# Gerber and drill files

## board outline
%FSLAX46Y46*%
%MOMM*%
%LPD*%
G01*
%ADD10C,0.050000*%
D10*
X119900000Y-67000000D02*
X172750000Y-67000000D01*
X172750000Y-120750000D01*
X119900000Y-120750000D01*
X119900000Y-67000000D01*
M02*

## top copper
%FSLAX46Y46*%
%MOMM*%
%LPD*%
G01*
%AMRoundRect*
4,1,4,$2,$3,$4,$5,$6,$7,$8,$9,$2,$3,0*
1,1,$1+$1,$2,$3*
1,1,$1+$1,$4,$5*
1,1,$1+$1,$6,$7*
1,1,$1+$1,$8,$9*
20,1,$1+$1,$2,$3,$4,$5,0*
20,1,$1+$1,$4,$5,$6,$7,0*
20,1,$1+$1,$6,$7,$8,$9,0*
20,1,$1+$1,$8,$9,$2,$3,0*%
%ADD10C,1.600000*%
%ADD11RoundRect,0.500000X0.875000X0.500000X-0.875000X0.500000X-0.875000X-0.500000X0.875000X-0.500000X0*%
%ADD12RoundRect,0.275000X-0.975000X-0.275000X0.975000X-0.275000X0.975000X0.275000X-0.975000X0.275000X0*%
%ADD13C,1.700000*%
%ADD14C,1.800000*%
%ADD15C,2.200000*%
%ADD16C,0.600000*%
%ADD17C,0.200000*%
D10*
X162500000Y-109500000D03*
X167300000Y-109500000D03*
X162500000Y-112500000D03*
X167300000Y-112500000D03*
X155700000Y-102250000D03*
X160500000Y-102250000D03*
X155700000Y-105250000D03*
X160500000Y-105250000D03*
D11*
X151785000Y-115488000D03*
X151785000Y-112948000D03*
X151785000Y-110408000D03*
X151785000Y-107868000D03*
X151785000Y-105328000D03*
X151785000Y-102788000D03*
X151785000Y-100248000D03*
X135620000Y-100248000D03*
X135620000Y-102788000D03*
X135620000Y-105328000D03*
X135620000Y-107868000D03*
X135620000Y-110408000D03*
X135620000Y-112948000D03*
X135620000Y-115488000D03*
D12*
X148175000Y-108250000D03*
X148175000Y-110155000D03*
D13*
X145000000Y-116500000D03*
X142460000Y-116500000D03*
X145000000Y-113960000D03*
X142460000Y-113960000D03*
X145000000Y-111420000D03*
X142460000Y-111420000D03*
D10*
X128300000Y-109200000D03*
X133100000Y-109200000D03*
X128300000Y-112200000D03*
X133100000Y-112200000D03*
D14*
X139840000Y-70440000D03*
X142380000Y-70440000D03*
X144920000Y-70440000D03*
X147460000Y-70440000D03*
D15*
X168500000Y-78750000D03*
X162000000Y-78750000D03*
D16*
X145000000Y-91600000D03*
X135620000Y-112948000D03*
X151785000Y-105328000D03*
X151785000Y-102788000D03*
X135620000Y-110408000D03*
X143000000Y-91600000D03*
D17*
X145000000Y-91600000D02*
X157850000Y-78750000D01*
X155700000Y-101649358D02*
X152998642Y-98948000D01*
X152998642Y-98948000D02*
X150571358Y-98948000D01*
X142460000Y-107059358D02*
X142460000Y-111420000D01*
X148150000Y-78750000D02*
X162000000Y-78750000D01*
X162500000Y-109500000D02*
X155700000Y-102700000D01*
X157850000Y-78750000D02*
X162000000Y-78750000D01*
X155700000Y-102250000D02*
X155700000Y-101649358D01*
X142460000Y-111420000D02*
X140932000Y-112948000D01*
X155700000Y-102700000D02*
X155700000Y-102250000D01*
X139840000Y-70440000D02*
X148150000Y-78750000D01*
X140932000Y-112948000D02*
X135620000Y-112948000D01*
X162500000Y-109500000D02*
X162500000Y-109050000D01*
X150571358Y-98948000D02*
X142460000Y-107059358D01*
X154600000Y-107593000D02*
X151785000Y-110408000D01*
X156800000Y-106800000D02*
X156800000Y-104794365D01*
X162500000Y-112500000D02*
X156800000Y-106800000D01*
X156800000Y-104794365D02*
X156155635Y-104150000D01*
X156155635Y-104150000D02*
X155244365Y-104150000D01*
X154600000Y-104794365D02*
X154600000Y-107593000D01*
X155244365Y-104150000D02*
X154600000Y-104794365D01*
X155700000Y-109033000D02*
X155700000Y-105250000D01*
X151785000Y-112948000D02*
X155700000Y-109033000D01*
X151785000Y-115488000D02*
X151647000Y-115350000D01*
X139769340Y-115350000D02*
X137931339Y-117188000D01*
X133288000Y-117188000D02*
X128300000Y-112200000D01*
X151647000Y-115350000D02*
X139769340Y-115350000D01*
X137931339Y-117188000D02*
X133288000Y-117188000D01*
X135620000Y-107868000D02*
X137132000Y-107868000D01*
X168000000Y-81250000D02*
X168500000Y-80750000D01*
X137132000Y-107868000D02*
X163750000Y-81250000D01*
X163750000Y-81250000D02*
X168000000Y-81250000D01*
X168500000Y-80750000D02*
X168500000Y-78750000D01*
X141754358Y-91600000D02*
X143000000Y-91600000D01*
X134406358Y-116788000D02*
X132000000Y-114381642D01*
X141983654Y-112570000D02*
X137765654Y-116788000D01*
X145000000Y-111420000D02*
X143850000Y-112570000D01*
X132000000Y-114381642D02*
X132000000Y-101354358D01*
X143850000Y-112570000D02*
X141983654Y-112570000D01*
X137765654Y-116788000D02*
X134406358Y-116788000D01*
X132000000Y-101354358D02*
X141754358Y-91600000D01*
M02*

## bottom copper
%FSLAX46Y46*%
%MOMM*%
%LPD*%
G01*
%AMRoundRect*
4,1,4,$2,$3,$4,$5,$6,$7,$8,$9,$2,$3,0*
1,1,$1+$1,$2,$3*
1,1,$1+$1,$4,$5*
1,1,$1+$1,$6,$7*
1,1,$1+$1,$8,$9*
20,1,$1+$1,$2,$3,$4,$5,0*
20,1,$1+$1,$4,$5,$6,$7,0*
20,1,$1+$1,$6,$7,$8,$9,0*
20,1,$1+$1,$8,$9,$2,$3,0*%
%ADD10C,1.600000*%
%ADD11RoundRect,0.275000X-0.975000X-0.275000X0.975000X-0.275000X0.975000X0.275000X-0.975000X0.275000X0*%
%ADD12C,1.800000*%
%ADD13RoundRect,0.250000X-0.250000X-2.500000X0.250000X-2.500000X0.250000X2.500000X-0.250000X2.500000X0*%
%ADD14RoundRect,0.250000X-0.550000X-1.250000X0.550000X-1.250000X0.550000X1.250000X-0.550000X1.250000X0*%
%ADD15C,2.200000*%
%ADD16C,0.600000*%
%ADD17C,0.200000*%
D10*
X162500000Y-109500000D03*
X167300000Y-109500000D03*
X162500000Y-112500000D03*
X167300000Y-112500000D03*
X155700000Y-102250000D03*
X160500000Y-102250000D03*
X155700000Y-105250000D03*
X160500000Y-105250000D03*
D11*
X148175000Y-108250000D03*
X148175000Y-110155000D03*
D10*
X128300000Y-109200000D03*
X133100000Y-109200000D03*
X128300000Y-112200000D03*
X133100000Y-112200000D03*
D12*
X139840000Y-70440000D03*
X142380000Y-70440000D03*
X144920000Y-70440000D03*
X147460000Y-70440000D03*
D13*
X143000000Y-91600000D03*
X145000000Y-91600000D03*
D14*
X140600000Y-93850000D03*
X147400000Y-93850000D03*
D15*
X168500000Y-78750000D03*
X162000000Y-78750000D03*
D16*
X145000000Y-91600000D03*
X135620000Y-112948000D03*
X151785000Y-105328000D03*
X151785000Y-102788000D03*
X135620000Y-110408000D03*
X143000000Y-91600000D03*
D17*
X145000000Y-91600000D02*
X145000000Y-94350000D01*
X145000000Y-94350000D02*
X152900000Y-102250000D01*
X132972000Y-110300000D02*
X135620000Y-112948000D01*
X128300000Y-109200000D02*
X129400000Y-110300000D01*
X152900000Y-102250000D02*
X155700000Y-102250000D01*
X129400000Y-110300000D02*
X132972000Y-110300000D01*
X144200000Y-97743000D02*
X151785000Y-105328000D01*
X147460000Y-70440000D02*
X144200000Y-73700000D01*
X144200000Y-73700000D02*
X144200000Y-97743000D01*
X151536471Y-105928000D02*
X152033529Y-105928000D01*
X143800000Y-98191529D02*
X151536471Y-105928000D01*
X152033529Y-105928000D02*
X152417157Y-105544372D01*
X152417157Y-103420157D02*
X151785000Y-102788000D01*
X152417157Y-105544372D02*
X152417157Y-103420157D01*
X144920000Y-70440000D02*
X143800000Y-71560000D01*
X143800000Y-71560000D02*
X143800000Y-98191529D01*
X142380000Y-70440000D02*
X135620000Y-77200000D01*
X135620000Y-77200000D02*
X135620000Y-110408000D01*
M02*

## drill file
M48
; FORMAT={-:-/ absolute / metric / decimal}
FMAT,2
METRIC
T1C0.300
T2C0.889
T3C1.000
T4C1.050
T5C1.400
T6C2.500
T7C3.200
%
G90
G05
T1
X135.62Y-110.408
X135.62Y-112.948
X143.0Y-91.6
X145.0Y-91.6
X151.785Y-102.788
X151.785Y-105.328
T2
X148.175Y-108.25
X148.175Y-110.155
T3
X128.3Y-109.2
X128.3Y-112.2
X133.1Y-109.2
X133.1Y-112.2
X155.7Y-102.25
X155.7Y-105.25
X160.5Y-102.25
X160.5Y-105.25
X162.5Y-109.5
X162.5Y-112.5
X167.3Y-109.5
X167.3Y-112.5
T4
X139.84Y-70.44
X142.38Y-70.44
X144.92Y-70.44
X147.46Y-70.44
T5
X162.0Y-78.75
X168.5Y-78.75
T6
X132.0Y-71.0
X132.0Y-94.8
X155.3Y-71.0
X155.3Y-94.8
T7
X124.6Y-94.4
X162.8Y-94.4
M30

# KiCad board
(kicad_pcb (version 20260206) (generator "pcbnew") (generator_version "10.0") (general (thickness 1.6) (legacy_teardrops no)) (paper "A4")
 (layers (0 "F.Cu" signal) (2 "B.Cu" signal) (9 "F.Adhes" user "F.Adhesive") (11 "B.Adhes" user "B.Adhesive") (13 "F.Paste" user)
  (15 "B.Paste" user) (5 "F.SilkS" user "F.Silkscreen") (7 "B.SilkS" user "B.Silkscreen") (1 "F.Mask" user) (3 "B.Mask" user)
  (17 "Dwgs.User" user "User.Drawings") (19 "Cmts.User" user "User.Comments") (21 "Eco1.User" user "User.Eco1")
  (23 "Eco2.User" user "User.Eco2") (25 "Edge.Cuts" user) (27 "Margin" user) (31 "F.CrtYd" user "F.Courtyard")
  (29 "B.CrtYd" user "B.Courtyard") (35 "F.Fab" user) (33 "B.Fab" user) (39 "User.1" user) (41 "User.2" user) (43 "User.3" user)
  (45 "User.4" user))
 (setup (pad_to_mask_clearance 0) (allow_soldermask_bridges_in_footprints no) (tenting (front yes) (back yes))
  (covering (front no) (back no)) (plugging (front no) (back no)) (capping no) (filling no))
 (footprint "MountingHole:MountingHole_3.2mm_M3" (layer "F.Cu") (at 162.8 94.4)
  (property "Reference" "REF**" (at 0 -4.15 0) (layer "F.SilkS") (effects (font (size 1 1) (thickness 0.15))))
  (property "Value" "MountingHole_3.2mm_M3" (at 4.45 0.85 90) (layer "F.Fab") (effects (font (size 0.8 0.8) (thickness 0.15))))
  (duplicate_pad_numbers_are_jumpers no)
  (pad "" np_thru_hole circle (at 0 0) (size 3.2 3.2) (drill 3.2) (layers "*.Cu" "*.Mask")))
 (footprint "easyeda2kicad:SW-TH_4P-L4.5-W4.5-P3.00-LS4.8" (layer "F.Cu") (at 164.9 111)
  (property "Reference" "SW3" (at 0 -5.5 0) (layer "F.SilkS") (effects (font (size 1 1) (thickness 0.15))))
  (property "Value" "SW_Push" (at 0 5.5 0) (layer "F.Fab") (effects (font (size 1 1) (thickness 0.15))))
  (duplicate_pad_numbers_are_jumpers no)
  (pad "1" thru_hole circle (at -2.4 -1.5) (size 1.6 1.6) (drill 0.999998) (layers "*.Cu" "*.Mask") (remove_unused_layers no) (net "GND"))
  (pad "1" thru_hole circle (at 2.4 -1.5) (size 1.6 1.6) (drill 0.999998) (layers "*.Cu" "*.Mask") (remove_unused_layers no))
  (pad "2" thru_hole circle (at -2.4 1.5) (size 1.6 1.6) (drill 0.999998) (layers "*.Cu" "*.Mask") (remove_unused_layers no)
   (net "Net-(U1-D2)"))
  (pad "2" thru_hole circle (at 2.4 1.5) (size 1.6 1.6) (drill 0.999998) (layers "*.Cu" "*.Mask") (remove_unused_layers no)))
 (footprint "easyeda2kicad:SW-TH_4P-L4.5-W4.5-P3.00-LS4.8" (layer "F.Cu") (at 158.1 103.75)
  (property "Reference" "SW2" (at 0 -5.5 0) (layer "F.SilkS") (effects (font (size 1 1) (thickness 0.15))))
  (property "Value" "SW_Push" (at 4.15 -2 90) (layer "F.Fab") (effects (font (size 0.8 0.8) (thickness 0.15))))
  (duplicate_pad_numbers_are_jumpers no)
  (pad "1" thru_hole circle (at -2.4 -1.5) (size 1.6 1.6) (drill 0.999998) (layers "*.Cu" "*.Mask") (remove_unused_layers no) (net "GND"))
  (pad "1" thru_hole circle (at 2.4 -1.5) (size 1.6 1.6) (drill 0.999998) (layers "*.Cu" "*.Mask") (remove_unused_layers no))
  (pad "2" thru_hole circle (at -2.4 1.5) (size 1.6 1.6) (drill 0.999998) (layers "*.Cu" "*.Mask") (remove_unused_layers no)
   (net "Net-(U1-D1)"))
  (pad "2" thru_hole circle (at 2.4 1.5) (size 1.6 1.6) (drill 0.999998) (layers "*.Cu" "*.Mask") (remove_unused_layers no)))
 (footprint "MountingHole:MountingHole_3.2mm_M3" (layer "F.Cu") (at 124.6 94.4)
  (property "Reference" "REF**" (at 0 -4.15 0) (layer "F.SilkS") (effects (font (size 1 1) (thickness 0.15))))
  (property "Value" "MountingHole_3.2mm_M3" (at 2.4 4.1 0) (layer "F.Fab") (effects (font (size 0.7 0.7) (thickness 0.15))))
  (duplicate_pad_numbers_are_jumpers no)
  (pad "" np_thru_hole circle (at 0 0) (size 3.2 3.2) (drill 3.2) (layers "*.Cu" "*.Mask")))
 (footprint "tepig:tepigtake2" (layer "F.Cu") (at 124.75 74.25)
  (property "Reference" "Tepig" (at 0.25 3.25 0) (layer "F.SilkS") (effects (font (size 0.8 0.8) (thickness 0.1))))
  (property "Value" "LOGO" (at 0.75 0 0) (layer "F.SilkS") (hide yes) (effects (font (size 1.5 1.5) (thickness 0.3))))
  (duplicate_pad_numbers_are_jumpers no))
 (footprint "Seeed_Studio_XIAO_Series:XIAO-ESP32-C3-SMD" (layer "F.Cu") (at 152.62 97.368 180)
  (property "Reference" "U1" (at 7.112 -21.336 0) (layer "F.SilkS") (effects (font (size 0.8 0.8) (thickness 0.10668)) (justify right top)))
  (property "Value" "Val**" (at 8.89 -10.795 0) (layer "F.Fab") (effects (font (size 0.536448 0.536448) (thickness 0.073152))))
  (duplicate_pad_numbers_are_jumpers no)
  (pad "1" smd roundrect (at 0.835 -18.12 180) (size 2.75 2) (layers "F.Cu" "F.Mask" "F.Paste") (roundrect_rratio 0.25) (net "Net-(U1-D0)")
   (solder_mask_margin 0.0508) (thermal_bridge_angle 45))
  (pad "2" smd roundrect (at 0.835 -15.58 180) (size 2.75 2) (layers "F.Cu" "F.Mask" "F.Paste") (roundrect_rratio 0.25) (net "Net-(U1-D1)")
   (solder_mask_margin 0.0508) (thermal_bridge_angle 45))
  (pad "3" smd roundrect (at 0.835 -13.04 180) (size 2.75 2) (layers "F.Cu" "F.Mask" "F.Paste") (roundrect_rratio 0.25) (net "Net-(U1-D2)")
   (solder_mask_margin 0.0508) (thermal_bridge_angle 45))
  (pad "4" smd roundrect (at 0.835 -10.5 180) (size 2.75 2) (layers "F.Cu" "F.Mask" "F.Paste") (roundrect_rratio 0.25)
   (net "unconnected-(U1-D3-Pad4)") (solder_mask_margin 0.0508) (thermal_bridge_angle 45))
  (pad "5" smd roundrect (at 0.835 -7.96 180) (size 2.75 2) (layers "F.Cu" "F.Mask" "F.Paste") (roundrect_rratio 0.25) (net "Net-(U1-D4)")
   (solder_mask_margin 0.0508) (thermal_bridge_angle 45))
  (pad "6" smd roundrect (at 0.835 -5.42 180) (size 2.75 2) (layers "F.Cu" "F.Mask" "F.Paste") (roundrect_rratio 0.25) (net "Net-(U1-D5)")
   (solder_mask_margin 0.0508) (thermal_bridge_angle 45))
  (pad "7" smd roundrect (at 0.835 -2.88 180) (size 2.75 2) (layers "F.Cu" "F.Mask" "F.Paste") (roundrect_rratio 0.25)
   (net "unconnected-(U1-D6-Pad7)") (solder_mask_margin 0.0508) (thermal_bridge_angle 45))
  (pad "8" smd roundrect (at 17 -2.88 180) (size 2.75 2) (layers "F.Cu" "F.Mask" "F.Paste") (roundrect_rratio 0.25)
   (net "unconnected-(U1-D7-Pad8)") (solder_mask_margin 0.0508) (thermal_bridge_angle 45))
  (pad "9" smd roundrect (at 17 -5.42 180) (size 2.75 2) (layers "F.Cu" "F.Mask" "F.Paste") (roundrect_rratio 0.25)
   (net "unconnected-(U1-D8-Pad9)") (solder_mask_margin 0.0508) (thermal_bridge_angle 45))
  (pad "10" smd roundrect (at 17 -7.96 180) (size 2.75 2) (layers "F.Cu" "F.Mask" "F.Paste") (roundrect_rratio 0.25)
   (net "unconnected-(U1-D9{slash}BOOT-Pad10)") (solder_mask_margin 0.0508) (thermal_bridge_angle 45))
  (pad "11" smd roundrect (at 17 -10.5 180) (size 2.75 2) (layers "F.Cu" "F.Mask" "F.Paste") (roundrect_rratio 0.25) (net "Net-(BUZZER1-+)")
   (solder_mask_margin 0.0508) (thermal_bridge_angle 45))
  (pad "12" smd roundrect (at 17 -13.04 180) (size 2.75 2) (layers "F.Cu" "F.Mask" "F.Paste") (roundrect_rratio 0.25) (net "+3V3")
   (solder_mask_margin 0.0508) (thermal_bridge_angle 45))
  (pad "13" smd roundrect (at 17 -15.58 180) (size 2.75 2) (layers "F.Cu" "F.Mask" "F.Paste") (roundrect_rratio 0.25) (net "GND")
   (solder_mask_margin 0.0508) (thermal_bridge_angle 45))
  (pad "14" smd roundrect (at 17 -18.12 180) (size 2.75 2) (layers "F.Cu" "F.Mask" "F.Paste") (roundrect_rratio 0.25) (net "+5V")
   (solder_mask_margin 0.0508) (thermal_bridge_angle 45))
  (pad "15" thru_hole roundrect (at 4.445 -10.882) (size 2.5 1.1) (drill 0.889) (layers "*.Cu" "*.Mask") (remove_unused_layers no)
   (roundrect_rratio 0.25) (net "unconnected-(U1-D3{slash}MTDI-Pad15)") (thermal_bridge_angle 45))
  (pad "16" thru_hole roundrect (at 4.445 -12.787) (size 2.5 1.1) (drill 0.889) (layers "*.Cu" "*.Mask") (remove_unused_layers no)
   (roundrect_rratio 0.25) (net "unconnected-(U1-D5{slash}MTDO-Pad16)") (thermal_bridge_angle 45))
  (pad "17" smd circle (at 7.62 -19.132 180) (size 1.7 1.7) (layers "F.Cu" "F.Mask" "F.Paste") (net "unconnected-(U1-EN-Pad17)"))
  (pad "18" smd circle (at 10.16 -19.132 180) (size 1.7 1.7) (layers "F.Cu" "F.Mask" "F.Paste") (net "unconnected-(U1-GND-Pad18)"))
  (pad "19" smd circle (at 7.62 -16.592 180) (size 1.7 1.7) (layers "F.Cu" "F.Mask" "F.Paste") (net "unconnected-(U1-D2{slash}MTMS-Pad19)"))
  (pad "20" smd circle (at 10.16 -16.592 180) (size 1.7 1.7) (layers "F.Cu" "F.Mask" "F.Paste") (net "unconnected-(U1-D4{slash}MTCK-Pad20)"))
  (pad "21" smd circle (at 7.62 -14.052 180) (size 1.7 1.7) (layers "F.Cu" "F.Mask" "F.Paste") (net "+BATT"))
  (pad "22" smd circle (at 10.16 -14.052 180) (size 1.7 1.7) (layers "F.Cu" "F.Mask" "F.Paste") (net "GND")))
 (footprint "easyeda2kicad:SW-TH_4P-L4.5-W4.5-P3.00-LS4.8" (layer "F.Cu") (at 130.7 110.7)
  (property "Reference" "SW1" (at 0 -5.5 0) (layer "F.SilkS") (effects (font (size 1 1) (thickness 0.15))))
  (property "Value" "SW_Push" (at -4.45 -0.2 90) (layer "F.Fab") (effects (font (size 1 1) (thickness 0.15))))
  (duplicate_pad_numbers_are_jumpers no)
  (pad "1" thru_hole circle (at -2.4 -1.5) (size 1.6 1.6) (drill 0.999998) (layers "*.Cu" "*.Mask") (remove_unused_layers no) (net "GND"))
  (pad "1" thru_hole circle (at 2.4 -1.5) (size 1.6 1.6) (drill 0.999998) (layers "*.Cu" "*.Mask") (remove_unused_layers no))
  (pad "2" thru_hole circle (at -2.4 1.5) (size 1.6 1.6) (drill 0.999998) (layers "*.Cu" "*.Mask") (remove_unused_layers no)
   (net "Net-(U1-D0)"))
  (pad "2" thru_hole circle (at 2.4 1.5) (size 1.6 1.6) (drill 0.999998) (layers "*.Cu" "*.Mask") (remove_unused_layers no)))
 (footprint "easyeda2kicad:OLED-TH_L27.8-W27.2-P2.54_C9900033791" (layer "F.Cu") (at 143.65 70.44)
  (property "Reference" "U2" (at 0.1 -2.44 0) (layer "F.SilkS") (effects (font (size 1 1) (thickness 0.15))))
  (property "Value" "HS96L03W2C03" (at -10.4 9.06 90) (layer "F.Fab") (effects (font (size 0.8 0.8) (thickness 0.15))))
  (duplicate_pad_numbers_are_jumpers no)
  (pad "" np_thru_hole circle (at -11.65 0.56) (size 2.5 2.5) (drill 2.5) (layers "*.Cu" "*.Mask"))
  (pad "" np_thru_hole circle (at -11.65 24.36) (size 2.5 2.5) (drill 2.5) (layers "*.Cu" "*.Mask"))
  (pad "" np_thru_hole circle (at 11.65 0.56) (size 2.5 2.5) (drill 2.5) (layers "*.Cu" "*.Mask"))
  (pad "" np_thru_hole circle (at 11.65 24.36) (size 2.5 2.5) (drill 2.5) (layers "*.Cu" "*.Mask"))
  (pad "1" thru_hole circle (at -3.81 0) (size 1.8 1.8) (drill 1.049986) (layers "*.Cu" "*.Mask") (remove_unused_layers no) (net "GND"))
  (pad "2" thru_hole circle (at -1.27 0) (size 1.8 1.8) (drill 1.049986) (layers "*.Cu" "*.Mask") (remove_unused_layers no) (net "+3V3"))
  (pad "3" thru_hole circle (at 1.27 0) (size 1.8 1.8) (drill 1.049986) (layers "*.Cu" "*.Mask") (remove_unused_layers no)
   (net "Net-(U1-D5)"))
  (pad "4" thru_hole circle (at 3.81 0) (size 1.8 1.8) (drill 1.049986) (layers "*.Cu" "*.Mask") (remove_unused_layers no)
   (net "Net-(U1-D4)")))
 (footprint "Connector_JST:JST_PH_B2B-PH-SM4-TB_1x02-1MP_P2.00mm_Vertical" (layer "B.Cu") (at 144 92.1)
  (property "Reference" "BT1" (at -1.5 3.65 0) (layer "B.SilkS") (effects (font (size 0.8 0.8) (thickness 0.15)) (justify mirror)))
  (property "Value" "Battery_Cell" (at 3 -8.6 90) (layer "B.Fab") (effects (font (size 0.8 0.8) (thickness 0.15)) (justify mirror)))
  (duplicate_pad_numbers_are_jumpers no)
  (pad "1" smd roundrect (at -1 -0.5) (size 1 5.5) (layers "B.Cu" "B.Mask" "B.Paste") (roundrect_rratio 0.25) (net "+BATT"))
  (pad "2" smd roundrect (at 1 -0.5) (size 1 5.5) (layers "B.Cu" "B.Mask" "B.Paste") (roundrect_rratio 0.25) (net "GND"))
  (pad "MP" smd roundrect (at -3.4 1.75) (size 1.6 3) (layers "B.Cu" "B.Mask" "B.Paste") (roundrect_rratio 0.15625))
  (pad "MP" smd roundrect (at 3.4 1.75) (size 1.6 3) (layers "B.Cu" "B.Mask" "B.Paste") (roundrect_rratio 0.15625)))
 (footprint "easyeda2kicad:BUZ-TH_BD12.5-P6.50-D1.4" (layer "B.Cu") (at 165.25 78.75 180)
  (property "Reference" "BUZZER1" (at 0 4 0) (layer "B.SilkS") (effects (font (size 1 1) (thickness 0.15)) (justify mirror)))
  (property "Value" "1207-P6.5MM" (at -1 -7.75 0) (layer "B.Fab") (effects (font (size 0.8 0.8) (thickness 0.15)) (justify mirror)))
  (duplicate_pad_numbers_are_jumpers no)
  (pad "1" thru_hole circle (at -3.25 0 180) (size 2.2 2.2) (drill 1.399998) (layers "*.Cu" "*.Mask") (remove_unused_layers no)
   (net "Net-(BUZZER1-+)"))
  (pad "2" thru_hole circle (at 3.25 0 180) (size 2.2 2.2) (drill 1.399998) (layers "*.Cu" "*.Mask") (remove_unused_layers no) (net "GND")))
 (gr_rect (start 119.9 67) (end 172.75 120.75) (stroke (width 0.05) (type default)) (fill no) (layer "Edge.Cuts"))
 (segment (start 145 91.6) (end 157.85 78.75) (width 0.2) (layer "F.Cu") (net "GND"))
 (segment (start 155.7 101.649358) (end 152.998642 98.948) (width 0.2) (layer "F.Cu") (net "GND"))
 (segment (start 152.998642 98.948) (end 150.571358 98.948) (width 0.2) (layer "F.Cu") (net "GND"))
 (segment (start 142.46 107.059358) (end 142.46 111.42) (width 0.2) (layer "F.Cu") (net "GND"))
 (segment (start 148.15 78.75) (end 162 78.75) (width 0.2) (layer "F.Cu") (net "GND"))
 (segment (start 162.5 109.5) (end 155.7 102.7) (width 0.2) (layer "F.Cu") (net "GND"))
 (segment (start 157.85 78.75) (end 162 78.75) (width 0.2) (layer "F.Cu") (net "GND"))
 (segment (start 155.7 102.25) (end 155.7 101.649358) (width 0.2) (layer "F.Cu") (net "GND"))
 (segment (start 142.46 111.42) (end 140.932 112.948) (width 0.2) (layer "F.Cu") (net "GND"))
 (segment (start 155.7 102.7) (end 155.7 102.25) (width 0.2) (layer "F.Cu") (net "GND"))
 (segment (start 139.84 70.44) (end 148.15 78.75) (width 0.2) (layer "F.Cu") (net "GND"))
 (segment (start 140.932 112.948) (end 135.62 112.948) (width 0.2) (layer "F.Cu") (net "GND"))
 (segment (start 162.5 109.5) (end 162.5 109.05) (width 0.2) (layer "F.Cu") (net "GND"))
 (segment (start 150.571358 98.948) (end 142.46 107.059358) (width 0.2) (layer "F.Cu") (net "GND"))
 (via (at 145 91.6) (size 0.6) (drill 0.3) (layers "F.Cu" "B.Cu") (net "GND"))
 (via (at 135.62 112.948) (size 0.6) (drill 0.3) (layers "F.Cu" "B.Cu") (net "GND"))
 (segment (start 145 91.6) (end 145 94.35) (width 0.2) (layer "B.Cu") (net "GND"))
 (segment (start 145 94.35) (end 152.9 102.25) (width 0.2) (layer "B.Cu") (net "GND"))
 (segment (start 132.972 110.3) (end 135.62 112.948) (width 0.2) (layer "B.Cu") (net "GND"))
 (segment (start 128.3 109.2) (end 129.4 110.3) (width 0.2) (layer "B.Cu") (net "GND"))
 (segment (start 152.9 102.25) (end 155.7 102.25) (width 0.2) (layer "B.Cu") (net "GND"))
 (segment (start 129.4 110.3) (end 132.972 110.3) (width 0.2) (layer "B.Cu") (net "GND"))
 (segment (start 154.6 107.593) (end 151.785 110.408) (width 0.2) (layer "F.Cu") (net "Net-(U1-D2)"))
 (segment (start 156.8 106.8) (end 156.8 104.794365) (width 0.2) (layer "F.Cu") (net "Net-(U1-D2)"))
 (segment (start 162.5 112.5) (end 156.8 106.8) (width 0.2) (layer "F.Cu") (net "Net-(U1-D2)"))
 (segment (start 156.8 104.794365) (end 156.155635 104.15) (width 0.2) (layer "F.Cu") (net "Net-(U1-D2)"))
 (segment (start 156.155635 104.15) (end 155.244365 104.15) (width 0.2) (layer "F.Cu") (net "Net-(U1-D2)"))
 (segment (start 154.6 104.794365) (end 154.6 107.593) (width 0.2) (layer "F.Cu") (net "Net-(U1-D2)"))
 (segment (start 155.244365 104.15) (end 154.6 104.794365) (width 0.2) (layer "F.Cu") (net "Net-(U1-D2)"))
 (segment (start 155.7 109.033) (end 155.7 105.25) (width 0.2) (layer "F.Cu") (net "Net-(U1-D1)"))
 (segment (start 151.785 112.948) (end 155.7 109.033) (width 0.2) (layer "F.Cu") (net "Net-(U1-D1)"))
 (segment (start 151.785 115.488) (end 151.647 115.35) (width 0.2) (layer "F.Cu") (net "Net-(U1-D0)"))
 (segment (start 139.76934 115.35) (end 137.931339 117.188) (width 0.2) (layer "F.Cu") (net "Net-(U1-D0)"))
 (segment (start 133.288 117.188) (end 128.3 112.2) (width 0.2) (layer "F.Cu") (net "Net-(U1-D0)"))
 (segment (start 151.647 115.35) (end 139.76934 115.35) (width 0.2) (layer "F.Cu") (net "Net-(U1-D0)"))
 (segment (start 137.931339 117.188) (end 133.288 117.188) (width 0.2) (layer "F.Cu") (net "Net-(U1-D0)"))
 (via (at 151.785 105.328) (size 0.6) (drill 0.3) (layers "F.Cu" "B.Cu") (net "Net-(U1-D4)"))
 (segment (start 144.2 97.743) (end 151.785 105.328) (width 0.2) (layer "B.Cu") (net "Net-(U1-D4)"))
 (segment (start 147.46 70.44) (end 144.2 73.7) (width 0.2) (layer "B.Cu") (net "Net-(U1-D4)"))
 (segment (start 144.2 73.7) (end 144.2 97.743) (width 0.2) (layer "B.Cu") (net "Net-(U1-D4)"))
 (via (at 151.785 102.788) (size 0.6) (drill 0.3) (layers "F.Cu" "B.Cu") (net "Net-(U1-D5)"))
 (segment (start 151.536471 105.928) (end 152.033529 105.928) (width 0.2) (layer "B.Cu") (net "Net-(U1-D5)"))
 (segment (start 143.8 98.191529) (end 151.536471 105.928) (width 0.2) (layer "B.Cu") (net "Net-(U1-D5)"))
 (segment (start 152.033529 105.928) (end 152.417157 105.544372) (width 0.2) (layer "B.Cu") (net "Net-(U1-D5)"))
 (segment (start 152.417157 103.420157) (end 151.785 102.788) (width 0.2) (layer "B.Cu") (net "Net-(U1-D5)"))
 (segment (start 152.417157 105.544372) (end 152.417157 103.420157) (width 0.2) (layer "B.Cu") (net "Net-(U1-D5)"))
 (segment (start 144.92 70.44) (end 143.8 71.56) (width 0.2) (layer "B.Cu") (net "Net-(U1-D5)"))
 (segment (start 143.8 71.56) (end 143.8 98.191529) (width 0.2) (layer "B.Cu") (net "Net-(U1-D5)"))
 (segment (start 135.62 107.868) (end 137.132 107.868) (width 0.2) (layer "F.Cu") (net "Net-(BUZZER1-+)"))
 (segment (start 168 81.25) (end 168.5 80.75) (width 0.2) (layer "F.Cu") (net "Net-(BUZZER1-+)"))
 (segment (start 137.132 107.868) (end 163.75 81.25) (width 0.2) (layer "F.Cu") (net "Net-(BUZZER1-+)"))
 (segment (start 163.75 81.25) (end 168 81.25) (width 0.2) (layer "F.Cu") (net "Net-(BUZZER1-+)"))
 (segment (start 168.5 80.75) (end 168.5 78.75) (width 0.2) (layer "F.Cu") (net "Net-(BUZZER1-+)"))
 (via (at 135.62 110.408) (size 0.6) (drill 0.3) (layers "F.Cu" "B.Cu") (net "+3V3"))
 (segment (start 142.38 70.44) (end 135.62 77.2) (width 0.2) (layer "B.Cu") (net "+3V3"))
 (segment (start 135.62 77.2) (end 135.62 110.408) (width 0.2) (layer "B.Cu") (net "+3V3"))
 (segment (start 141.754358 91.6) (end 143 91.6) (width 0.2) (layer "F.Cu") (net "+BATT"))
 (segment (start 134.406358 116.788) (end 132 114.381642) (width 0.2) (layer "F.Cu") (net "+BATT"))
 (segment (start 141.983654 112.57) (end 137.765654 116.788) (width 0.2) (layer "F.Cu") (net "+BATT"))
 (segment (start 145 111.42) (end 143.85 112.57) (width 0.2) (layer "F.Cu") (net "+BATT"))
 (segment (start 132 114.381642) (end 132 101.354358) (width 0.2) (layer "F.Cu") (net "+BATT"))
 (segment (start 143.85 112.57) (end 141.983654 112.57) (width 0.2) (layer "F.Cu") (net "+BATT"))
 (segment (start 137.765654 116.788) (end 134.406358 116.788) (width 0.2) (layer "F.Cu") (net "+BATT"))
 (segment (start 132 101.354358) (end 141.754358 91.6) (width 0.2) (layer "F.Cu") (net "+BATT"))
 (via (at 143 91.6) (size 0.6) (drill 0.3) (layers "F.Cu" "B.Cu") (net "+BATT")))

